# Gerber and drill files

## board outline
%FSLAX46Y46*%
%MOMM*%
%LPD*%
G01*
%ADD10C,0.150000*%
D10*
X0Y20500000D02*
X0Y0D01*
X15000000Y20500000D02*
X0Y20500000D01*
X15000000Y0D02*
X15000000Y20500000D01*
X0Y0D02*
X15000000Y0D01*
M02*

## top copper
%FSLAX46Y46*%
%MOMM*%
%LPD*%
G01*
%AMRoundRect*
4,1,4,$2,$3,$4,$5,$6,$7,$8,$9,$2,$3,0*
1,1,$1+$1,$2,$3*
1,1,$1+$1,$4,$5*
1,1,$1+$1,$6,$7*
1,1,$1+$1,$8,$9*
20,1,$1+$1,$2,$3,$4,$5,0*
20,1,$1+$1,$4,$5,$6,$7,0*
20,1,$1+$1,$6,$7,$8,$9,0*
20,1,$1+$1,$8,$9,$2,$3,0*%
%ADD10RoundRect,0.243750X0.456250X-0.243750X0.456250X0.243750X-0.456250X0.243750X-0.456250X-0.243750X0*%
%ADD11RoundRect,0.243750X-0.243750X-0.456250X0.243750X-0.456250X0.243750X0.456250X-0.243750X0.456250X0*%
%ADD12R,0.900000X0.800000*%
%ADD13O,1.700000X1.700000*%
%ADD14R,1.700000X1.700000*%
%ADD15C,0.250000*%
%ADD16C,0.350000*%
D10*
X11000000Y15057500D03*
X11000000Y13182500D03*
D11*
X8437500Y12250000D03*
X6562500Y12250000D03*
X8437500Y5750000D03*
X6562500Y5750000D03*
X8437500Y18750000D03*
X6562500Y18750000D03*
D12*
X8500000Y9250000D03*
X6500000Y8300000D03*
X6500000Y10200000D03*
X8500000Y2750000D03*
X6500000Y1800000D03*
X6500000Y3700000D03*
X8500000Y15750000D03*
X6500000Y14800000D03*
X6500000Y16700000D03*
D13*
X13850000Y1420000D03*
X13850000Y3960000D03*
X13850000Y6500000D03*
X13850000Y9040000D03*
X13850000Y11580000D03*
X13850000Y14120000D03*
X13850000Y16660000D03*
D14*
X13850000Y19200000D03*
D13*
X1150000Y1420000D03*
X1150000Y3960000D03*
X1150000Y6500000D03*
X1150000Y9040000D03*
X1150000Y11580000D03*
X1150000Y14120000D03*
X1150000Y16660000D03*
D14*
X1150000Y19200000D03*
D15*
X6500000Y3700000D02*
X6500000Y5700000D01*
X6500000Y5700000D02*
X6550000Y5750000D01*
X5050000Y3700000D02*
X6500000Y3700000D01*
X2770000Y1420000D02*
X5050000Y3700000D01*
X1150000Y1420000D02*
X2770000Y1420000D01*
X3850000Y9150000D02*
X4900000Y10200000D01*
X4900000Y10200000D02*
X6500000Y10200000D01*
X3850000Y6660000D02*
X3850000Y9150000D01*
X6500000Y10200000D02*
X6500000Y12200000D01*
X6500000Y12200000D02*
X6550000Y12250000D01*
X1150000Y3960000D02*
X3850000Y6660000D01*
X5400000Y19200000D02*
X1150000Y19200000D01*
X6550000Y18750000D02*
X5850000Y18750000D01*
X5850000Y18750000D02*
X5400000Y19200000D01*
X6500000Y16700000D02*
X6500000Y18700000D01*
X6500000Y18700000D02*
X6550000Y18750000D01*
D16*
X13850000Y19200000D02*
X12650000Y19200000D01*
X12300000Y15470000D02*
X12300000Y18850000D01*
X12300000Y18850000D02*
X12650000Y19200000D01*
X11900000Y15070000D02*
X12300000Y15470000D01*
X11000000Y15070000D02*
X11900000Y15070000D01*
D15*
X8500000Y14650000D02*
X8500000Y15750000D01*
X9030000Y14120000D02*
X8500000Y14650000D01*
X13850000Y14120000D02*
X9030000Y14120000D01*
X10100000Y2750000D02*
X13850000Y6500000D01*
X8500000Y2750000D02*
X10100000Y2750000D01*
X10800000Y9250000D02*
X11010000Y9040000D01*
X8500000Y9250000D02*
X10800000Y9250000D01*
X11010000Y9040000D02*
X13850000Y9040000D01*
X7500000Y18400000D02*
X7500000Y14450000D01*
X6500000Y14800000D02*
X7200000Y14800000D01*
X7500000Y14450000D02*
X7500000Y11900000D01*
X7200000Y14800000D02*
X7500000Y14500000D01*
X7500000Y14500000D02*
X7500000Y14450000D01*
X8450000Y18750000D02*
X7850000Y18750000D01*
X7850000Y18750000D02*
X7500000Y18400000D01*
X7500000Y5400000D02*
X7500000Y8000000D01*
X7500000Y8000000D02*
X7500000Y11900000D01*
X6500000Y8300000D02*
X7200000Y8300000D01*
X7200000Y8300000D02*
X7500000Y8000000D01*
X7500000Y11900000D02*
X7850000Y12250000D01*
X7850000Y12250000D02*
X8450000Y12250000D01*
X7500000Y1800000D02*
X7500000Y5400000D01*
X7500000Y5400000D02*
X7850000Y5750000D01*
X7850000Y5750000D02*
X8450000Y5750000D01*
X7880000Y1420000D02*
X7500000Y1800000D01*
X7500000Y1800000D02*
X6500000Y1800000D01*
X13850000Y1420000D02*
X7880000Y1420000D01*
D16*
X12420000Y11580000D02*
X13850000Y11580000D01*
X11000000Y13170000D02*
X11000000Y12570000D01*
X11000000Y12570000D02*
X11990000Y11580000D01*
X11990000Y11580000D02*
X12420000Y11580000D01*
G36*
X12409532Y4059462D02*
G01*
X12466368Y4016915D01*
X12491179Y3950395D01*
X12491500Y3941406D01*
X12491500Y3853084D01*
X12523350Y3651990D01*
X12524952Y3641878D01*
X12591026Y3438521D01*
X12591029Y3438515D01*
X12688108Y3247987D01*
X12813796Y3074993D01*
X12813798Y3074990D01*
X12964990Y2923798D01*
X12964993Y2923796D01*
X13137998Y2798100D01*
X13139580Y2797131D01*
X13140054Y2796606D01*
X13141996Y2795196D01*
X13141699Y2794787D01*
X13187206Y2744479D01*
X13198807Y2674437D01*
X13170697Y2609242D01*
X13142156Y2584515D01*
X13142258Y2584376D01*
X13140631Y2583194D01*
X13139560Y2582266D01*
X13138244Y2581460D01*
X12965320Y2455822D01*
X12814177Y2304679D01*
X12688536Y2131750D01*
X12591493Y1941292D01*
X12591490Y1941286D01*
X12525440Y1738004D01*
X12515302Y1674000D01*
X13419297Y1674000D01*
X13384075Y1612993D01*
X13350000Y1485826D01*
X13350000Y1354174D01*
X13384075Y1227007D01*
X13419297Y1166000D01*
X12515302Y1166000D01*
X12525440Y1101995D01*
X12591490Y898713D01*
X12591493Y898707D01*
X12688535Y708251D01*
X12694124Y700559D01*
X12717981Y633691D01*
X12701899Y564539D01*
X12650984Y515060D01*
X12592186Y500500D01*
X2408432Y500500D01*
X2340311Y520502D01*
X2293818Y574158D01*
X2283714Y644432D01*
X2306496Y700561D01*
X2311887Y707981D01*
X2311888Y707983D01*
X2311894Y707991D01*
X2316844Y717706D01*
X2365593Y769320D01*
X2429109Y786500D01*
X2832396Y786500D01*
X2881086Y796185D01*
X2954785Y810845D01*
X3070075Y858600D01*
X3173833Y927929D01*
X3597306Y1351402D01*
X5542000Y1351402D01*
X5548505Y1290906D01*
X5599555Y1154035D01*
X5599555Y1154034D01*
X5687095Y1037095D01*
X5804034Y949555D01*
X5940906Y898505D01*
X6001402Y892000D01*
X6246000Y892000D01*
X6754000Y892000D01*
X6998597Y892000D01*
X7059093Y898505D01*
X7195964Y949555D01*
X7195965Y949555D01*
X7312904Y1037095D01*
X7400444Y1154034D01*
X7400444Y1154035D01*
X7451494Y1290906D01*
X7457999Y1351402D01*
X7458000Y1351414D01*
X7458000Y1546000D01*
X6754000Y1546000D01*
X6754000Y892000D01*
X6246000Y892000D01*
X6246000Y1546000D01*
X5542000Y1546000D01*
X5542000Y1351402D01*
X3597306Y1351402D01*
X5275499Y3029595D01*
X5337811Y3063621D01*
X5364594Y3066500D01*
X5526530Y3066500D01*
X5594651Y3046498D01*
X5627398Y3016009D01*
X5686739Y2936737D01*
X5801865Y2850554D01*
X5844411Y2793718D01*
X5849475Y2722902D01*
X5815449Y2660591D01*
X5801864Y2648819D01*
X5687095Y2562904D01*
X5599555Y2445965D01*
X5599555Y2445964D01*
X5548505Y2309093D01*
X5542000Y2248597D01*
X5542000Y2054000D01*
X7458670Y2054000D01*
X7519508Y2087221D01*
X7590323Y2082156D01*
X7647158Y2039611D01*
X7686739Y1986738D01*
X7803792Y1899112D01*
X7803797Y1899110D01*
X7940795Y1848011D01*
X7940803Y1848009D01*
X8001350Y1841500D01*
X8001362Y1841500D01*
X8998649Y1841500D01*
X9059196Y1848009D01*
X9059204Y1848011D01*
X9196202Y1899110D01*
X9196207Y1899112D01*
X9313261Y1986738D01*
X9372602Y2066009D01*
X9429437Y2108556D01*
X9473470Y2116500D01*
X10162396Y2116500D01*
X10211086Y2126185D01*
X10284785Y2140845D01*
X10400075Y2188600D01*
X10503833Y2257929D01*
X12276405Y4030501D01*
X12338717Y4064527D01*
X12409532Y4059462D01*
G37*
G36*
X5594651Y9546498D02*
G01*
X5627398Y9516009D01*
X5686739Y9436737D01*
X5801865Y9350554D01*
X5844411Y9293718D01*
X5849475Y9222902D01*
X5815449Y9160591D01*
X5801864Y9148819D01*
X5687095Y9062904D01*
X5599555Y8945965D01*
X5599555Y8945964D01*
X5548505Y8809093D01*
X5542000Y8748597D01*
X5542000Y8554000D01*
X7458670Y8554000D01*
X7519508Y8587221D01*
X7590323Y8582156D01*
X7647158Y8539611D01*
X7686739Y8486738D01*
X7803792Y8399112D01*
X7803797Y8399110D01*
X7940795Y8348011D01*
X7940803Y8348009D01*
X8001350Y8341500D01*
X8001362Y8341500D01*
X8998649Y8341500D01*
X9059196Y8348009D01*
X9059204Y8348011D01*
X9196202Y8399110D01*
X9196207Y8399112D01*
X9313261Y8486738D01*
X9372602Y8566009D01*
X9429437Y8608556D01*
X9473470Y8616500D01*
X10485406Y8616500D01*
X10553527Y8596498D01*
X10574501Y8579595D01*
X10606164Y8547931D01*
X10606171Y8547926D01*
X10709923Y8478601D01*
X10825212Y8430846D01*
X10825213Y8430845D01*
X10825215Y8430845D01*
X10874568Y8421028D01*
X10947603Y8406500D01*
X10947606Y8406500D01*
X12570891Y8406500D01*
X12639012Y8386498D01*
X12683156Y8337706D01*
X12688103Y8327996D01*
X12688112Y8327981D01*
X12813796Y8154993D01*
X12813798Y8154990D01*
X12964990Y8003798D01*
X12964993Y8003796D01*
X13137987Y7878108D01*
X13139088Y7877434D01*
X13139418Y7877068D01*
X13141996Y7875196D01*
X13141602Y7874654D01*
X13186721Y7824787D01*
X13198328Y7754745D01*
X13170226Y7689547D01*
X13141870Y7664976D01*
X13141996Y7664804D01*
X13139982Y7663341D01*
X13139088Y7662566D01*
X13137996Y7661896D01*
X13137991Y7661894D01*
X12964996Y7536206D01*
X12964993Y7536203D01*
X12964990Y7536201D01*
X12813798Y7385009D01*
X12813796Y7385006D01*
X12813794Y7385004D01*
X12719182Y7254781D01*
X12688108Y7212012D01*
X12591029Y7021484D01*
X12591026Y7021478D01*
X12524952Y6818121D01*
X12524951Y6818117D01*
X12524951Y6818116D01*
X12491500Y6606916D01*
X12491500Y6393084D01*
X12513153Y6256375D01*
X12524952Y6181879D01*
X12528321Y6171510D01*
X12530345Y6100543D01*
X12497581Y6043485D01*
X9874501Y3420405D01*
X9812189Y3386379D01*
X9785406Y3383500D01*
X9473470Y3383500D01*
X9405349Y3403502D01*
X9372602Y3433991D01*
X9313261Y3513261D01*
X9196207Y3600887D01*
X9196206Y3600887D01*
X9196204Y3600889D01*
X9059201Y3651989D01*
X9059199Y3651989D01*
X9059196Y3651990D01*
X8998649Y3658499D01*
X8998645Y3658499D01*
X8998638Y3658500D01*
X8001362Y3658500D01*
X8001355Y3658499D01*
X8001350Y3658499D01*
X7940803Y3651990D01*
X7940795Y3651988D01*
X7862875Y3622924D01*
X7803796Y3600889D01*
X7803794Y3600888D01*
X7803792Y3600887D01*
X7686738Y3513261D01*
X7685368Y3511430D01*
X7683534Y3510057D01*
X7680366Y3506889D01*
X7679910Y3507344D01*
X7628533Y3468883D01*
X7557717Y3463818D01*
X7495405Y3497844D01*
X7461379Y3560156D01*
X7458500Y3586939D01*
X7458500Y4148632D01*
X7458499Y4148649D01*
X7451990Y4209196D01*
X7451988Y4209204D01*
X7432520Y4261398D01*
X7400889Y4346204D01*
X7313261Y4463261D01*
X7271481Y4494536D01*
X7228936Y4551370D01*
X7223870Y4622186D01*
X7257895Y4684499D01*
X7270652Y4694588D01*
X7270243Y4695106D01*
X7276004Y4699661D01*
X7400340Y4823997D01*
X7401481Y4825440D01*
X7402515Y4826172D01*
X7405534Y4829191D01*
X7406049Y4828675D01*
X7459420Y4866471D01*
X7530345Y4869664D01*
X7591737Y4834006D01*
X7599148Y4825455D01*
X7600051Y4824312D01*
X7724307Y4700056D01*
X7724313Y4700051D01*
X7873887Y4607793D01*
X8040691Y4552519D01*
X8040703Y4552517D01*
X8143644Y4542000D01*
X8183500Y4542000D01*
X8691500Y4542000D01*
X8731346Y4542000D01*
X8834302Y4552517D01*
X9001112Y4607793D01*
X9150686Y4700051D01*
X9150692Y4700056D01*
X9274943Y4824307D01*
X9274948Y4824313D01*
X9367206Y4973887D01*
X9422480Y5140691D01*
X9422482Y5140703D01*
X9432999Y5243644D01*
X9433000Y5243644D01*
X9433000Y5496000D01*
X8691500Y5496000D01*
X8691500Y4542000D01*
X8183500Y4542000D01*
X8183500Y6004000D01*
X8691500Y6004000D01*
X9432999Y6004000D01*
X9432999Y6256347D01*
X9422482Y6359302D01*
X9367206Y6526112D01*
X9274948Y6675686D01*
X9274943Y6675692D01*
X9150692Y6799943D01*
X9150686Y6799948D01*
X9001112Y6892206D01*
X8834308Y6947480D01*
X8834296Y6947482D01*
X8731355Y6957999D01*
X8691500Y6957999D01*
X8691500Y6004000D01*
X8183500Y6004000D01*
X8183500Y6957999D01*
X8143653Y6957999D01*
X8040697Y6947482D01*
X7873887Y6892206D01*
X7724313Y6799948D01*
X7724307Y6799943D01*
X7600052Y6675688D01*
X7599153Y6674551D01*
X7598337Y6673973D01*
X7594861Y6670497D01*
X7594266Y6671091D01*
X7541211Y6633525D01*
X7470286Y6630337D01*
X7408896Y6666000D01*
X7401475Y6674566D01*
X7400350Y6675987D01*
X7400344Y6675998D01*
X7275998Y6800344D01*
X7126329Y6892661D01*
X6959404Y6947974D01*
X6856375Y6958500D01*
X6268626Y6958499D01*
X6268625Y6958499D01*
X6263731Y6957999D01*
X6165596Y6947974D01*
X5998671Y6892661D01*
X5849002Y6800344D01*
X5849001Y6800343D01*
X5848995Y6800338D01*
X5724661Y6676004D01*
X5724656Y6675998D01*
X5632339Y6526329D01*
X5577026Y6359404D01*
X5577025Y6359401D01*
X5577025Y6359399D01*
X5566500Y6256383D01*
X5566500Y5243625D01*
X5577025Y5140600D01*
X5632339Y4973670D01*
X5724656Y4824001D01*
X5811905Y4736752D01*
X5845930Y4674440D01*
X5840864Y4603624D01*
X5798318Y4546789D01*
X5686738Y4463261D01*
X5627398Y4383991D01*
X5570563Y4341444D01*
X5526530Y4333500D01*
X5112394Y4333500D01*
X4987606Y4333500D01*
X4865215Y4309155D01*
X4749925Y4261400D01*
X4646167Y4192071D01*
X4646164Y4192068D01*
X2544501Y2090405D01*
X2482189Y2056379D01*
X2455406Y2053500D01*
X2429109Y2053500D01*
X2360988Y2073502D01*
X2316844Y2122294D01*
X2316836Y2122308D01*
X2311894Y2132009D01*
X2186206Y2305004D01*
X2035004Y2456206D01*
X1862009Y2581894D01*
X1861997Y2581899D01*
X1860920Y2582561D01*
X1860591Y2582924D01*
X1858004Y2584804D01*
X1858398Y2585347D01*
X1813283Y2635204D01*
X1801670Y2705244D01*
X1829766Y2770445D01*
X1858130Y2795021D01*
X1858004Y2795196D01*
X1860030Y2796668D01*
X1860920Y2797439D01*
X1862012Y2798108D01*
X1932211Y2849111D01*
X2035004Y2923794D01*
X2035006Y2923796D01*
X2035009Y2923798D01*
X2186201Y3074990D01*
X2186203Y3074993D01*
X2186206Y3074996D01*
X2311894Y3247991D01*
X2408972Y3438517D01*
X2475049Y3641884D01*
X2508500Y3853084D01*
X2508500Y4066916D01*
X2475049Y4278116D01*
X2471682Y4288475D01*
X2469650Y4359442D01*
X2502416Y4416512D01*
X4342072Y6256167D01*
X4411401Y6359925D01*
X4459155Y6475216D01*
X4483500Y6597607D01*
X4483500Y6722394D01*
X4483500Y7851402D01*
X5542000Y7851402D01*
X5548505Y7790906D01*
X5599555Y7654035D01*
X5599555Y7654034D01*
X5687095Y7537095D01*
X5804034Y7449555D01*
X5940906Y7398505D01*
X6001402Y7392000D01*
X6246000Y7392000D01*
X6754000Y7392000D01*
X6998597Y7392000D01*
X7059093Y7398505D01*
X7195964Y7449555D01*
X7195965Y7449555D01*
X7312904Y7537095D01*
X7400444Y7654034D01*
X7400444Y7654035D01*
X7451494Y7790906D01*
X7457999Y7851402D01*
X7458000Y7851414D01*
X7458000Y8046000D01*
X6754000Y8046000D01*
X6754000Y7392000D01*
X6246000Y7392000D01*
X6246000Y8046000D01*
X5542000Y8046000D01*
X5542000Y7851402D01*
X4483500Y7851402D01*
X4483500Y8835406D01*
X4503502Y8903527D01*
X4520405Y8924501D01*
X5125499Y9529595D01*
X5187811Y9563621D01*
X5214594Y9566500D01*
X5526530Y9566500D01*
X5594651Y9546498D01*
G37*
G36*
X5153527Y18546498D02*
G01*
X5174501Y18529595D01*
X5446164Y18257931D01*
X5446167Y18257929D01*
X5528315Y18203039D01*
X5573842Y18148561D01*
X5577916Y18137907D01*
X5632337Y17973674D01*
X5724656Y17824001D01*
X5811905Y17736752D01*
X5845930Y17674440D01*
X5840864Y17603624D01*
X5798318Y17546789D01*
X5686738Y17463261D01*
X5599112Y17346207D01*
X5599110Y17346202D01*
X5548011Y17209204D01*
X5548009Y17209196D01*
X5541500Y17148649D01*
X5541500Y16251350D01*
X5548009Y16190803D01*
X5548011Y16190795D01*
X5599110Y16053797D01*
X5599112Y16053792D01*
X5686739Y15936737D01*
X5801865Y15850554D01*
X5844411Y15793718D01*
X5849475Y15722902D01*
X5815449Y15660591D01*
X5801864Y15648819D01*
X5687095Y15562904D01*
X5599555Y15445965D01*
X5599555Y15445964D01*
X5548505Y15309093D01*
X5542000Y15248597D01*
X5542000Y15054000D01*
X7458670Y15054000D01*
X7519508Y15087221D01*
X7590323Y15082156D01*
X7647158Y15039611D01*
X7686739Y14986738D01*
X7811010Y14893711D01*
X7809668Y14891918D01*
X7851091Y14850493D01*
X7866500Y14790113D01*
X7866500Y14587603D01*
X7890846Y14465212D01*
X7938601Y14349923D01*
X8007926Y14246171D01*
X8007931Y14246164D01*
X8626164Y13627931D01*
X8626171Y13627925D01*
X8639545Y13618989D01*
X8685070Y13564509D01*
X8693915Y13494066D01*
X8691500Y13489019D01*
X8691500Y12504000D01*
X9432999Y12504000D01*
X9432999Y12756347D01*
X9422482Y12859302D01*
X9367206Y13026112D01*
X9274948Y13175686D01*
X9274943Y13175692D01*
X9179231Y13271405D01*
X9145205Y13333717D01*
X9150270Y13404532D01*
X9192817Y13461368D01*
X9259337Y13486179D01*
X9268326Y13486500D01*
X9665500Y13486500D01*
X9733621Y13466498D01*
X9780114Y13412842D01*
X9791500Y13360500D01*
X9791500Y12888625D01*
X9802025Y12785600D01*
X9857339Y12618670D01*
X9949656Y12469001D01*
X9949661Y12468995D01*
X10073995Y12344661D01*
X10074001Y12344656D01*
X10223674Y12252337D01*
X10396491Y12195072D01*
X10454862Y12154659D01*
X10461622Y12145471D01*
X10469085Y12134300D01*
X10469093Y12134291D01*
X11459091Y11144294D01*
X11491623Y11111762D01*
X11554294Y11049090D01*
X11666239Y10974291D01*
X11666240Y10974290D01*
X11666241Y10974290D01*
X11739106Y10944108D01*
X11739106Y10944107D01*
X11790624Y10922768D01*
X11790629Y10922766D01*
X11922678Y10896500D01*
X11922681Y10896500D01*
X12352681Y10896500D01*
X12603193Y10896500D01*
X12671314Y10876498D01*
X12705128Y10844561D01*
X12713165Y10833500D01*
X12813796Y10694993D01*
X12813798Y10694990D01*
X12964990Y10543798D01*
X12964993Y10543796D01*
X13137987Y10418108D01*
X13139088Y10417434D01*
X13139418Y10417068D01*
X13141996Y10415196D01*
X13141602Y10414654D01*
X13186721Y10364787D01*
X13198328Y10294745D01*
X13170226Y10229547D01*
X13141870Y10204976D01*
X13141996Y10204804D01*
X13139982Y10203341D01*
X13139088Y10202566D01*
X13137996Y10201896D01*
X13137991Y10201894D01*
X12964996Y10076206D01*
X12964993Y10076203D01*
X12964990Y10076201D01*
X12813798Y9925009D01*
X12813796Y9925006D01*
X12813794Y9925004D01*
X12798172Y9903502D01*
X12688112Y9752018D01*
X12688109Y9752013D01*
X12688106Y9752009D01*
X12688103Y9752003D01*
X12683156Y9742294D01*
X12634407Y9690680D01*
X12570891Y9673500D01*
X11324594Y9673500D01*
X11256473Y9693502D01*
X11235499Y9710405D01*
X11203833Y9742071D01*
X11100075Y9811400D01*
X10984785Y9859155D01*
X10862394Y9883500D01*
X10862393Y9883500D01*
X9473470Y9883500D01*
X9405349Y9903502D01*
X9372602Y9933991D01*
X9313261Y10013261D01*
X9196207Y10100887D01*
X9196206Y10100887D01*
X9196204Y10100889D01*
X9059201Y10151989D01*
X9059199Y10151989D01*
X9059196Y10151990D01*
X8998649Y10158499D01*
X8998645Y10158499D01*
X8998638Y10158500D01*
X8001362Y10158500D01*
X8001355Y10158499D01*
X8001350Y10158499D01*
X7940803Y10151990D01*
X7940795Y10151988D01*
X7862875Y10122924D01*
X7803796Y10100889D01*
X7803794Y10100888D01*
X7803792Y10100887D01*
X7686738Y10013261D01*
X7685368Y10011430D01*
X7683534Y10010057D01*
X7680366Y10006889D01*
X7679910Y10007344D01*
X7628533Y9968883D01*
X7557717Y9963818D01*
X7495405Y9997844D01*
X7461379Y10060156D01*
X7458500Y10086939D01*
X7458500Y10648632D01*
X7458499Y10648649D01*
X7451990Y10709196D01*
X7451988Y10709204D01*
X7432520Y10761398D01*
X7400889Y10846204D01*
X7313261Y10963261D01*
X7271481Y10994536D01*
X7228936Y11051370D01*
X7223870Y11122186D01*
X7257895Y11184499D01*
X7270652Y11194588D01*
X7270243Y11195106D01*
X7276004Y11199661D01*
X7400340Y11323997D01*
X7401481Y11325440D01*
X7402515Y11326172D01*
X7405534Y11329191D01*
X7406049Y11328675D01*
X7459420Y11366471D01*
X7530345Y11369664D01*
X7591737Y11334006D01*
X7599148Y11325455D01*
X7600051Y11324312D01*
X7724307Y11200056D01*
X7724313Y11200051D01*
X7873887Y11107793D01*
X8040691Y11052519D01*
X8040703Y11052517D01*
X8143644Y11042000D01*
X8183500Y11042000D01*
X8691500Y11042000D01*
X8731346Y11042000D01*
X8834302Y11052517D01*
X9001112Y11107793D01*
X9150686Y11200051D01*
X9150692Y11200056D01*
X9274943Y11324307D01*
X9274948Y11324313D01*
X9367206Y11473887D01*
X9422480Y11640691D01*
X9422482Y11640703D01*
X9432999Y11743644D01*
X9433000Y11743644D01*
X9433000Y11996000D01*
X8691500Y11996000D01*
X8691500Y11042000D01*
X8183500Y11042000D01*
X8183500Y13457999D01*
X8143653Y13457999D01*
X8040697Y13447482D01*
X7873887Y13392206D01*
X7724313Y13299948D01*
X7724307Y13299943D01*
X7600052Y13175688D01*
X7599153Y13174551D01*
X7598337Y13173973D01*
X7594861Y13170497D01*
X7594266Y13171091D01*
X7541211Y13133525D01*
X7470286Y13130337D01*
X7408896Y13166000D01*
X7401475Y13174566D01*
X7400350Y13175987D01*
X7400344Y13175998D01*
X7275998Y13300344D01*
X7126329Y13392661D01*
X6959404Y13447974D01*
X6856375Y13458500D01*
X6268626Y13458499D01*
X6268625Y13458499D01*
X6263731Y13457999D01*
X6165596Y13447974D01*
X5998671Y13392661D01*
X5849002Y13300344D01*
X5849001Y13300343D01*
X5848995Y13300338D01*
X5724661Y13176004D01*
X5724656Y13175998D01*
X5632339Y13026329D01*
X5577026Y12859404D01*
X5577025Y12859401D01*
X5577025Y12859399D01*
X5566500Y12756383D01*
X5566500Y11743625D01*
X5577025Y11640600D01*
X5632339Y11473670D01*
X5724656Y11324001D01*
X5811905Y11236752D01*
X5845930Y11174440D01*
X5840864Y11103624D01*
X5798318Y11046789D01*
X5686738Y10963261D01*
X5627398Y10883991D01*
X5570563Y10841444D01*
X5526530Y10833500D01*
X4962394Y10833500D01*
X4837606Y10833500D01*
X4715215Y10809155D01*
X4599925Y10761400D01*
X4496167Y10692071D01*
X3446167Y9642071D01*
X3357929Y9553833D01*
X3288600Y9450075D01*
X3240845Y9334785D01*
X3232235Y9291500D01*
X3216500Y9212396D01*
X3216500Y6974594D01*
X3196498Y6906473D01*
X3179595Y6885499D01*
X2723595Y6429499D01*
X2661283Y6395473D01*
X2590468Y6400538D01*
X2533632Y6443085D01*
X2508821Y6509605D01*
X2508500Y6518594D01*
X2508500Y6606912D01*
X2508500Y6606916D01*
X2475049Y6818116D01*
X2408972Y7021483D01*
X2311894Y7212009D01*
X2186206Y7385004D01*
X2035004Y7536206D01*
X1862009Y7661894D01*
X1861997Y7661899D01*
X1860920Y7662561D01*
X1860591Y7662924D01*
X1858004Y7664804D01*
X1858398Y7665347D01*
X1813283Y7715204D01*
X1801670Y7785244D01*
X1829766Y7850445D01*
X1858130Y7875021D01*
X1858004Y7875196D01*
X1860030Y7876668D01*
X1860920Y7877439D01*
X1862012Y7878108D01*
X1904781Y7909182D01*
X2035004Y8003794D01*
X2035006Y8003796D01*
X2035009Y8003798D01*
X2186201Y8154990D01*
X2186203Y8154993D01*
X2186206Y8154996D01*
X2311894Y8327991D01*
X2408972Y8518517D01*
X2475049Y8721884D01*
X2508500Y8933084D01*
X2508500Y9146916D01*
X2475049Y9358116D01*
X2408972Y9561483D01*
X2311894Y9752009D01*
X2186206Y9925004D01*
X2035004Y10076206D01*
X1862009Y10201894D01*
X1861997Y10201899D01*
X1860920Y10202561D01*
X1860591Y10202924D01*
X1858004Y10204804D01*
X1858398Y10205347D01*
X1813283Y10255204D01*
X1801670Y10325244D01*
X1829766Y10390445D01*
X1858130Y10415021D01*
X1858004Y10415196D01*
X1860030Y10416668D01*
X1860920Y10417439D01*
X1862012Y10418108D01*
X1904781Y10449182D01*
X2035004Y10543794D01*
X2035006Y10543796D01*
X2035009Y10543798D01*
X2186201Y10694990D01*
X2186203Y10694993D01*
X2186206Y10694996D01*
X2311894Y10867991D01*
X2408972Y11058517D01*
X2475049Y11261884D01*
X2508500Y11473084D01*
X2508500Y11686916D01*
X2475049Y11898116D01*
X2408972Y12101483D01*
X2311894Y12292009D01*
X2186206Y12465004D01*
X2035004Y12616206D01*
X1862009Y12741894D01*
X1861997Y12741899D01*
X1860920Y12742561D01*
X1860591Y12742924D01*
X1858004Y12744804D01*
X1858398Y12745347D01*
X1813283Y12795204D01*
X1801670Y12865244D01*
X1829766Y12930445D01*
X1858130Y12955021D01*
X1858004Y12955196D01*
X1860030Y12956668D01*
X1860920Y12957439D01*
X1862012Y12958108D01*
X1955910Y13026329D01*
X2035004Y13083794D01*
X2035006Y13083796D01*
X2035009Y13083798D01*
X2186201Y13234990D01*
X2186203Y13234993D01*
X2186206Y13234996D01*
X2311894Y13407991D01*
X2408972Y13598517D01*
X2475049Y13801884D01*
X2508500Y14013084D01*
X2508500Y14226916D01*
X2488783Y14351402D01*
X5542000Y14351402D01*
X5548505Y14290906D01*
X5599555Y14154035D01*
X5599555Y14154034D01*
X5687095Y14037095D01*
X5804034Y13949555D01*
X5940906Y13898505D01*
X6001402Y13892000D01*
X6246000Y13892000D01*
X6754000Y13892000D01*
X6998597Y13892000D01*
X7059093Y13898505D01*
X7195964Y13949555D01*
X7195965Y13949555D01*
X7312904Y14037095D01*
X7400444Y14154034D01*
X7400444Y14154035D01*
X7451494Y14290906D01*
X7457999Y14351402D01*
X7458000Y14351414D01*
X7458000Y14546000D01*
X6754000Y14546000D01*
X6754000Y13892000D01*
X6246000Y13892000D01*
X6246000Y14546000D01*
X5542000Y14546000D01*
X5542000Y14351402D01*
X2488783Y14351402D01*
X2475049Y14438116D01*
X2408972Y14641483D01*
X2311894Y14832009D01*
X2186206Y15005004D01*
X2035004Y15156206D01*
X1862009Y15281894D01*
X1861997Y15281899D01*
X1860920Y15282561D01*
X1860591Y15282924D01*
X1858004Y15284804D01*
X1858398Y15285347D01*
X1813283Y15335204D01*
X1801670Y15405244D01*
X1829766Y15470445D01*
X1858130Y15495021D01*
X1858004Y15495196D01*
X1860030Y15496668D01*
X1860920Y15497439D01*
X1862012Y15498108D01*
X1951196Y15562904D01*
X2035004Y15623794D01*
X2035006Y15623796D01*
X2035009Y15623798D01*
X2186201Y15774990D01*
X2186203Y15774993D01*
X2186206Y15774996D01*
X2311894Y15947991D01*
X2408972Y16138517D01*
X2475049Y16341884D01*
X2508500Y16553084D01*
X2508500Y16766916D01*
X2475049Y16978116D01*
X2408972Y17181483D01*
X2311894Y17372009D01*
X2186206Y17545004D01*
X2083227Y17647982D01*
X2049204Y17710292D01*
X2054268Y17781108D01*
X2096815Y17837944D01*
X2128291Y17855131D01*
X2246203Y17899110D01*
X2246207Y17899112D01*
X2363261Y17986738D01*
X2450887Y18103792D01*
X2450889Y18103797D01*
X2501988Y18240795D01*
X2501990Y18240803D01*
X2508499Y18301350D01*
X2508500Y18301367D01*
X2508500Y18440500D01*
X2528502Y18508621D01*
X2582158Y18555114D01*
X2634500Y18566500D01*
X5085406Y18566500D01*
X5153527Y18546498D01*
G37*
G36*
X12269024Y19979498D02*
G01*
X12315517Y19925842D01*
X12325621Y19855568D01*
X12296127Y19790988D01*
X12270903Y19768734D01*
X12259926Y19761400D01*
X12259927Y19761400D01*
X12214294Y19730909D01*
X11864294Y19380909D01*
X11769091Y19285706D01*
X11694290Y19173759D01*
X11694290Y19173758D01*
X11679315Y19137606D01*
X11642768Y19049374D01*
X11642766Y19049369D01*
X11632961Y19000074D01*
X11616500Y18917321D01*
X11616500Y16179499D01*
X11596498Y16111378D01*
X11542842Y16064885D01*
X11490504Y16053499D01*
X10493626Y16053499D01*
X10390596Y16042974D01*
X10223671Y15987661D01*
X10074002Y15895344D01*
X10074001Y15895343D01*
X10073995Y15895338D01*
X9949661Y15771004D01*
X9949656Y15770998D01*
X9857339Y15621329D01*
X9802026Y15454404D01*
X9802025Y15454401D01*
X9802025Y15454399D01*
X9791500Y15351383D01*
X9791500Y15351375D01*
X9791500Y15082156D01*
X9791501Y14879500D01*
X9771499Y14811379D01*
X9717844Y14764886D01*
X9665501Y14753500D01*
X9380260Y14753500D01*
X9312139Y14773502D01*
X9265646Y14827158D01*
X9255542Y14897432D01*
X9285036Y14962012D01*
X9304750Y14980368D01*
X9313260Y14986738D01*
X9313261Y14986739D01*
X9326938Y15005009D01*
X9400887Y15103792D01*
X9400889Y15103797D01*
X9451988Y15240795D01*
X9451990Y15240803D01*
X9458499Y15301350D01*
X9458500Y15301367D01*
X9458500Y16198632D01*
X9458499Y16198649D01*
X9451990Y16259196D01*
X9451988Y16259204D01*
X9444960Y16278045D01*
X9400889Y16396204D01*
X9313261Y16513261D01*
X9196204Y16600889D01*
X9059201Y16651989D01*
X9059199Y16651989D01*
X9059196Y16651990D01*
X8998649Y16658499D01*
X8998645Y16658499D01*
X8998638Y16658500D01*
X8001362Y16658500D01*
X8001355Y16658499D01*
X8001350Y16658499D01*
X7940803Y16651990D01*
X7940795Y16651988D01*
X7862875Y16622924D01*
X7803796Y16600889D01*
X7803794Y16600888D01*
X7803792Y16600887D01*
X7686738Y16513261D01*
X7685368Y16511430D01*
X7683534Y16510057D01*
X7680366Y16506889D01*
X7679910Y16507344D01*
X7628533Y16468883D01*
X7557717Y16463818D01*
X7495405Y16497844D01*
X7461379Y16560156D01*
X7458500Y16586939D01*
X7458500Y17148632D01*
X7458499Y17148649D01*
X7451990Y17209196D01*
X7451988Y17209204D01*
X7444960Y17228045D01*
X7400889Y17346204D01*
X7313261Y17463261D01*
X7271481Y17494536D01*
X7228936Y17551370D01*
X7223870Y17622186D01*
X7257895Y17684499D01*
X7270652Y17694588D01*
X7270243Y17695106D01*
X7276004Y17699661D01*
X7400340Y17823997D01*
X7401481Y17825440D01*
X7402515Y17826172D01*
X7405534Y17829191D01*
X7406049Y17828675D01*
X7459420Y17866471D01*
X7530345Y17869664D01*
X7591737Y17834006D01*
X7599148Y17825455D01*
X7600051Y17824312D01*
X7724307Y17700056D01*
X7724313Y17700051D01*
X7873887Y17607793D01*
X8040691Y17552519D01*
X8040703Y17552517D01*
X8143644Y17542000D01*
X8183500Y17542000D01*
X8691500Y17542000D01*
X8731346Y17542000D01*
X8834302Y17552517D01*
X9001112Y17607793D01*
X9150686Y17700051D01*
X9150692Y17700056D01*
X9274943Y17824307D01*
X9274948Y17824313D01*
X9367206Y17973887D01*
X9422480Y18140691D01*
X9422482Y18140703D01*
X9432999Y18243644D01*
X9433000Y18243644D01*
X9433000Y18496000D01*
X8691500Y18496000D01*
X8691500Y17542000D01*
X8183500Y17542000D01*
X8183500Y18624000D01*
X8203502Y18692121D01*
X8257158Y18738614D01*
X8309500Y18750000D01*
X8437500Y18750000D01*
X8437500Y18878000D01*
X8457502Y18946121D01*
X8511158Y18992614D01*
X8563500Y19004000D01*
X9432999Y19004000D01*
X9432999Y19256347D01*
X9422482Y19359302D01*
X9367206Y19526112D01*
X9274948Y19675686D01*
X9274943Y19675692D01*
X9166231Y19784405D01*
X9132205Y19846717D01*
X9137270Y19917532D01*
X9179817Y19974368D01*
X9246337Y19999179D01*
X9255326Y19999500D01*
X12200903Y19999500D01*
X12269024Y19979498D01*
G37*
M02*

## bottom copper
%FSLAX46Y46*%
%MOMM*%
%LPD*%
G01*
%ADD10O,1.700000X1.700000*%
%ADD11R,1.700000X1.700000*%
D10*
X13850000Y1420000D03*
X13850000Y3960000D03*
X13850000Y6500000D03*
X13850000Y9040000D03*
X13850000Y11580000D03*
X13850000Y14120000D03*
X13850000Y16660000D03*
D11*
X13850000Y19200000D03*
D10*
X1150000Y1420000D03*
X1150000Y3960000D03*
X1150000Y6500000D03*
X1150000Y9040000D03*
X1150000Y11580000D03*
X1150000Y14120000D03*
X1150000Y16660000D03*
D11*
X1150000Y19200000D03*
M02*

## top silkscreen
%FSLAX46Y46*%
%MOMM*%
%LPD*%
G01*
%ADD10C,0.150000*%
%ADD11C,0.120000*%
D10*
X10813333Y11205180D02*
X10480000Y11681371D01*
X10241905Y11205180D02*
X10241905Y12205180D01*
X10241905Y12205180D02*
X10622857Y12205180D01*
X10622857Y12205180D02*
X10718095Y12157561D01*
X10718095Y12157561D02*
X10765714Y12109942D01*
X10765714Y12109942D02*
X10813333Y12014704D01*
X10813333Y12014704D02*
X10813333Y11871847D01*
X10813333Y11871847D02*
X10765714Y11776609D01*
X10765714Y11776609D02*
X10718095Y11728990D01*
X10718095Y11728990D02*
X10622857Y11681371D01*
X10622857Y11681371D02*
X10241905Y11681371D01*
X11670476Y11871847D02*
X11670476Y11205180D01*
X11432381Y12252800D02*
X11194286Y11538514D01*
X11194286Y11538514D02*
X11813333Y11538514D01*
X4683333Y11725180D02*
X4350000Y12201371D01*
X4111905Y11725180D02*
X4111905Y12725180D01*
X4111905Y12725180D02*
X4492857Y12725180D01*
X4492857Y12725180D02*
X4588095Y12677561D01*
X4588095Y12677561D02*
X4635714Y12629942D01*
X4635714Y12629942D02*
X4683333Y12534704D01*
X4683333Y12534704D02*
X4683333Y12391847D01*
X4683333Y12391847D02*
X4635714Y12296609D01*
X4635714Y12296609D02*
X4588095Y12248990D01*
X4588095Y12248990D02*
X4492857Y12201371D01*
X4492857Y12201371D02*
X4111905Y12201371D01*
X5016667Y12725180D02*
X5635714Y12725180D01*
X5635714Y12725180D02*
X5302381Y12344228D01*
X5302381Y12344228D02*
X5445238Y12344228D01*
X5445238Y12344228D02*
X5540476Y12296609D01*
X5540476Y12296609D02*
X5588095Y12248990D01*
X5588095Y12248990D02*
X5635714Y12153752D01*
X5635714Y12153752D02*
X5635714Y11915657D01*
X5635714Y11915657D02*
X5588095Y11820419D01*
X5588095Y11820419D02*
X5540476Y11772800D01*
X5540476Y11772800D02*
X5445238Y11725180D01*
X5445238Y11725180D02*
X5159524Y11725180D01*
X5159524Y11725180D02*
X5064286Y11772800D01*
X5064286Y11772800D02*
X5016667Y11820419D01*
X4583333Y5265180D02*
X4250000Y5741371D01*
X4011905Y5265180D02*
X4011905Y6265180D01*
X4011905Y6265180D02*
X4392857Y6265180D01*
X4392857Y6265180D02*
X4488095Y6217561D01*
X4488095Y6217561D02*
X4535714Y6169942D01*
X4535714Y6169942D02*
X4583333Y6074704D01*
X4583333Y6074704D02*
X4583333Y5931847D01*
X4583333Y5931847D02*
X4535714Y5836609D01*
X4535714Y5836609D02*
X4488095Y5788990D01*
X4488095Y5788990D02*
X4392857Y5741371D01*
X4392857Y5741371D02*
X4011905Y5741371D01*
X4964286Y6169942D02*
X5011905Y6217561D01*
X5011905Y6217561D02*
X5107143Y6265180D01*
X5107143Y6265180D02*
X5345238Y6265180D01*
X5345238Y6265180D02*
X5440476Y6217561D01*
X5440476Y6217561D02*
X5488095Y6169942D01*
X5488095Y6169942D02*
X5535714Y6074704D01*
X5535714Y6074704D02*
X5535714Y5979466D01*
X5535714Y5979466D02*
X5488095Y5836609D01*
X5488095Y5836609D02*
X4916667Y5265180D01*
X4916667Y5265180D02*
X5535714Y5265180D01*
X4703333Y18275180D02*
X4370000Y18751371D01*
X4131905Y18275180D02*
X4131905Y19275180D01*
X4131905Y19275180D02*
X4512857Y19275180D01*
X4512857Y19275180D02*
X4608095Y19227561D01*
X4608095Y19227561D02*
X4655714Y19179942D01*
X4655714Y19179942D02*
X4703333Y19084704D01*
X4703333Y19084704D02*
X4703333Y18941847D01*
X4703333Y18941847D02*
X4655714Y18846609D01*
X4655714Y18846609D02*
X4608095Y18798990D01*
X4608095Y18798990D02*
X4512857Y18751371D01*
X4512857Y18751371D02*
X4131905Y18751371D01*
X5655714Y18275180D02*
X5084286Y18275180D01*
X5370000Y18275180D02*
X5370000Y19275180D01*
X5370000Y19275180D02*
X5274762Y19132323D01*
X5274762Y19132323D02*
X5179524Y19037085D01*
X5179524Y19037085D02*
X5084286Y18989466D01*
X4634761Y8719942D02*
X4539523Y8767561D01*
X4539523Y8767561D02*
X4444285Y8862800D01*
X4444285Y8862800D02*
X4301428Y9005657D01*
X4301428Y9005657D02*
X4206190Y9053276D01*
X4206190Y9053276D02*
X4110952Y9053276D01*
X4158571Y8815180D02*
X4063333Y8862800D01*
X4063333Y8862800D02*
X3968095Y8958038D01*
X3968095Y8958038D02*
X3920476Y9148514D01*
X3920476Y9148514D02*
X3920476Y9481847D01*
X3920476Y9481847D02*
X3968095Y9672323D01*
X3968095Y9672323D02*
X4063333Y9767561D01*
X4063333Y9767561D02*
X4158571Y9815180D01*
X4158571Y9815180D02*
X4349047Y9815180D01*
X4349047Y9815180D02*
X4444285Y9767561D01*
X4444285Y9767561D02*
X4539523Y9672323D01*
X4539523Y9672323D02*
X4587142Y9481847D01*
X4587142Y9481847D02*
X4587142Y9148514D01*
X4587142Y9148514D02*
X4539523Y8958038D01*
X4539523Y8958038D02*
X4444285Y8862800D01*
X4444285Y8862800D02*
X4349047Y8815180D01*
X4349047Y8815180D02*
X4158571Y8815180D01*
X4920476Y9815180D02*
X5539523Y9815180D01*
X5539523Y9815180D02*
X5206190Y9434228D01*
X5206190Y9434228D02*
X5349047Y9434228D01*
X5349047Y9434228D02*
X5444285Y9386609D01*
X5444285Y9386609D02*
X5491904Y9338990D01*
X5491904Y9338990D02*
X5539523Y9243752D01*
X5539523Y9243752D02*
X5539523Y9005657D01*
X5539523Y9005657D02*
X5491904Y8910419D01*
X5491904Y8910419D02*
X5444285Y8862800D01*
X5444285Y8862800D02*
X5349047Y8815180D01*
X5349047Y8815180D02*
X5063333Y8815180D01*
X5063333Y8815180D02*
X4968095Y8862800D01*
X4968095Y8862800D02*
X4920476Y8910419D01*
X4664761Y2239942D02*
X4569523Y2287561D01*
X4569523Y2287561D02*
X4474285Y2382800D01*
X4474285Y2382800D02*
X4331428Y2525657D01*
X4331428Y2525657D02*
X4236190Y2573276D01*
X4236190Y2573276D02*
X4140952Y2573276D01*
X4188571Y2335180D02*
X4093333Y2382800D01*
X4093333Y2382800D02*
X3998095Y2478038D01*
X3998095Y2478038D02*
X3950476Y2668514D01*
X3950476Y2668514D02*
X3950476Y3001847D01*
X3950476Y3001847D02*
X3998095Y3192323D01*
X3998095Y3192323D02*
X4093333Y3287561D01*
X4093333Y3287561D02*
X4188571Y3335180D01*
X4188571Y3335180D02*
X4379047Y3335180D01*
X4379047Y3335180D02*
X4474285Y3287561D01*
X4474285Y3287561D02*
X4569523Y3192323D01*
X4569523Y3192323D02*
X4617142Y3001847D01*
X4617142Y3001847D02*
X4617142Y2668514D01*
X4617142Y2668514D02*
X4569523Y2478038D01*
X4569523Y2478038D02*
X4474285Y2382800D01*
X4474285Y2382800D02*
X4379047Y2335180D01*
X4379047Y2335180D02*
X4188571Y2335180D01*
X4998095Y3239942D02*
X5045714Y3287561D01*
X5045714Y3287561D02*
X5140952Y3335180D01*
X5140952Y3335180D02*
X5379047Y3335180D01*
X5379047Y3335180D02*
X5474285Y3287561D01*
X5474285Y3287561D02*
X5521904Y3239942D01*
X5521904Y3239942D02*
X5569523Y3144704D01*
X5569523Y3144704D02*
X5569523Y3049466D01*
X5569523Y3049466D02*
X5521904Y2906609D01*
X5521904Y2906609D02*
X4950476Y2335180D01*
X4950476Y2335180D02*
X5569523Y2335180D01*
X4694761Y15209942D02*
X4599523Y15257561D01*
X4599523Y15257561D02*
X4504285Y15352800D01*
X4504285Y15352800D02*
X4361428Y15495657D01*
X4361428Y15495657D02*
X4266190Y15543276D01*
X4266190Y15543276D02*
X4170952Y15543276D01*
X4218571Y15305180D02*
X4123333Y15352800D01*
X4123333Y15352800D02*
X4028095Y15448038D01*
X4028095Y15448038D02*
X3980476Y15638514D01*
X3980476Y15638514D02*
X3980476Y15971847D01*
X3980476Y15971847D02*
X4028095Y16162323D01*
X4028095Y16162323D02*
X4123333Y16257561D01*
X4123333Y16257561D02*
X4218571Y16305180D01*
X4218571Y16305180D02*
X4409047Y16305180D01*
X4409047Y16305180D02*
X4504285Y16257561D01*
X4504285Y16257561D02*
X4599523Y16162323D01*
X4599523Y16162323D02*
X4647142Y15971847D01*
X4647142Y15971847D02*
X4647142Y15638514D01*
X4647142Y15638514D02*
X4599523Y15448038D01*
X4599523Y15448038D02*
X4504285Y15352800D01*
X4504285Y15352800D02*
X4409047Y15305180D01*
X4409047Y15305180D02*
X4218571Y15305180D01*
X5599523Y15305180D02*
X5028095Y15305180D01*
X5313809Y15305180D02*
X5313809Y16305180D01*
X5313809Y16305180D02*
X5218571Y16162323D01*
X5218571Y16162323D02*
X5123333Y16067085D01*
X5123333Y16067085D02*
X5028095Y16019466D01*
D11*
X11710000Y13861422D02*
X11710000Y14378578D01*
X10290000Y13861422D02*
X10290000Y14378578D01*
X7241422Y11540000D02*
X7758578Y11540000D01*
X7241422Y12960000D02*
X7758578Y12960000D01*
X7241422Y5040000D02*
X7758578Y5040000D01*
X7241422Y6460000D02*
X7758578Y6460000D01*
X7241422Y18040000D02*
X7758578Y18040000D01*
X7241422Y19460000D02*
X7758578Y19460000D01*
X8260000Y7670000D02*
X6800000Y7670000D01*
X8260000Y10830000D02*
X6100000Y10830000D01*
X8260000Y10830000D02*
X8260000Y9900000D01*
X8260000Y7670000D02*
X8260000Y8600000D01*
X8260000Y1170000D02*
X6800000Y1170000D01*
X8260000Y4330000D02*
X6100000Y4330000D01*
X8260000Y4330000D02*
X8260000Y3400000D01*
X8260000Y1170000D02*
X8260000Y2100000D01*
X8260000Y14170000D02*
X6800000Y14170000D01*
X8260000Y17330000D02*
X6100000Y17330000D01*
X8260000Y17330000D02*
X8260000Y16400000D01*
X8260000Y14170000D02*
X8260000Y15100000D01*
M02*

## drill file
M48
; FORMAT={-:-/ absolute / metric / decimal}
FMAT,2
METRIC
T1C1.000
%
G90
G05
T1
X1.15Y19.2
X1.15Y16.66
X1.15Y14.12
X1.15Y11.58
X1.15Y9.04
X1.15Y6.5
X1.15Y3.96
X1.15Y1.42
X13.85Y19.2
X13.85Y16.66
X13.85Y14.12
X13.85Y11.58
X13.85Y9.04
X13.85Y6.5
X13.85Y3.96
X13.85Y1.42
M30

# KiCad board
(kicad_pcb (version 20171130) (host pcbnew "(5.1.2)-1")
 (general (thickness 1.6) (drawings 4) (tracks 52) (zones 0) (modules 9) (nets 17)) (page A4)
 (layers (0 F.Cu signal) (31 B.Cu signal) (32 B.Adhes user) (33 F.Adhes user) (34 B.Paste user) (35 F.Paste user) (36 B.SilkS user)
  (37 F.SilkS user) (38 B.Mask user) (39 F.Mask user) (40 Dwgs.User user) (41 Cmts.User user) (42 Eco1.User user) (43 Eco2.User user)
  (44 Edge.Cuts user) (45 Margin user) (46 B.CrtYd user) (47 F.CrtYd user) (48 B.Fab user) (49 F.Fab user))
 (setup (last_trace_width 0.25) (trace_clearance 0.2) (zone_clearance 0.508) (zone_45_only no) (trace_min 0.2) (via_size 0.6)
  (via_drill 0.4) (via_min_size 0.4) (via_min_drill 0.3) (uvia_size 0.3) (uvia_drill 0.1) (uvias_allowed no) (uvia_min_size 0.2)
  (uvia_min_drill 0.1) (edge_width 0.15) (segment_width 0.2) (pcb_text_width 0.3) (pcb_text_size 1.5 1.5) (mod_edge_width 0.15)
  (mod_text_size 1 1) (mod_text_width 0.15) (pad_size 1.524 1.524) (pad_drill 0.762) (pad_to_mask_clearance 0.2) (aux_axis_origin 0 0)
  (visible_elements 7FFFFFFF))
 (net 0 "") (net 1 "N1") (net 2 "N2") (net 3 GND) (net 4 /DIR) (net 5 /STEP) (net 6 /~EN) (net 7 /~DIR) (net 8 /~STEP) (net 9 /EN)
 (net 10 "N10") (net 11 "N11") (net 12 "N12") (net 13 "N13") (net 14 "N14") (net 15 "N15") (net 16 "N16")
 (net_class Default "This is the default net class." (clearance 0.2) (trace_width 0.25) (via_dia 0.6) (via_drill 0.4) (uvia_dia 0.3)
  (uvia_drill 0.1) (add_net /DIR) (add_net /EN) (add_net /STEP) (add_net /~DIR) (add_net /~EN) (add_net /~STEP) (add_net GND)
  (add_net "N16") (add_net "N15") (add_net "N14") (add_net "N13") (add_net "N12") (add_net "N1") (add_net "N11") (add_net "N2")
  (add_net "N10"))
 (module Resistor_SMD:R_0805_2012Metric (layer F.Cu) (at 11 -14.12 90)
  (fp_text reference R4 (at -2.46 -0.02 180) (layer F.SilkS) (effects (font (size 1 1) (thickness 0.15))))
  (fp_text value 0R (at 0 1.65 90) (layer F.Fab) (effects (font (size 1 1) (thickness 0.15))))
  (fp_line (start -0.258578 0.71) (end 0.258578 0.71) (layer F.SilkS) (width 0.12))
  (fp_line (start -0.258578 -0.71) (end 0.258578 -0.71) (layer F.SilkS) (width 0.12))
  (pad 2 smd roundrect (at 0.9375 0 90) (size 0.975 1.4) (layers F.Cu F.Paste F.Mask) (roundrect_rratio 0.25) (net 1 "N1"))
  (pad 1 smd roundrect (at -0.9375 0 90) (size 0.975 1.4) (layers F.Cu F.Paste F.Mask) (roundrect_rratio 0.25) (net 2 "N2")))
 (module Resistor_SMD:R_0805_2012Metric (layer F.Cu) (at 7.5 -12.25)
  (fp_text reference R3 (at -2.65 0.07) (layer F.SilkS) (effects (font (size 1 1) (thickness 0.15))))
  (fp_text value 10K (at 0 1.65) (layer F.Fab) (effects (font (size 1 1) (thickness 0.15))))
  (fp_line (start -0.258578 0.71) (end 0.258578 0.71) (layer F.SilkS) (width 0.12))
  (fp_line (start -0.258578 -0.71) (end 0.258578 -0.71) (layer F.SilkS) (width 0.12))
  (pad 2 smd roundrect (at 0.9375 0) (size 0.975 1.4) (layers F.Cu F.Paste F.Mask) (roundrect_rratio 0.25) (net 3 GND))
  (pad 1 smd roundrect (at -0.9375 0) (size 0.975 1.4) (layers F.Cu F.Paste F.Mask) (roundrect_rratio 0.25) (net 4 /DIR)))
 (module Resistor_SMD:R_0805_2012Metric (layer F.Cu) (at 7.5 -5.75)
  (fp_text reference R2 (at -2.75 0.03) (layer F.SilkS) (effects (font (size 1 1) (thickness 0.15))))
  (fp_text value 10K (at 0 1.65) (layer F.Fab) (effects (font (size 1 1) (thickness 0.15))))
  (fp_line (start -0.258578 0.71) (end 0.258578 0.71) (layer F.SilkS) (width 0.12))
  (fp_line (start -0.258578 -0.71) (end 0.258578 -0.71) (layer F.SilkS) (width 0.12))
  (pad 2 smd roundrect (at 0.9375 0) (size 0.975 1.4) (layers F.Cu F.Paste F.Mask) (roundrect_rratio 0.25) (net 3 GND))
  (pad 1 smd roundrect (at -0.9375 0) (size 0.975 1.4) (layers F.Cu F.Paste F.Mask) (roundrect_rratio 0.25) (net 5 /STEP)))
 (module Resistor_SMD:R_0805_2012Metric (layer F.Cu) (at 7.5 -18.75)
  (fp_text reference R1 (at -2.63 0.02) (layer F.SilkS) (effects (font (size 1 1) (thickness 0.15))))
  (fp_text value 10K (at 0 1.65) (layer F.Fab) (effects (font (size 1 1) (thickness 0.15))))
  (fp_line (start -0.258578 0.71) (end 0.258578 0.71) (layer F.SilkS) (width 0.12))
  (fp_line (start -0.258578 -0.71) (end 0.258578 -0.71) (layer F.SilkS) (width 0.12))
  (pad 2 smd roundrect (at 0.9375 0) (size 0.975 1.4) (layers F.Cu F.Paste F.Mask) (roundrect_rratio 0.25) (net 3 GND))
  (pad 1 smd roundrect (at -0.9375 0) (size 0.975 1.4) (layers F.Cu F.Paste F.Mask) (roundrect_rratio 0.25) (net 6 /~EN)))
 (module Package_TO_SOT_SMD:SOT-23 (layer F.Cu) (at 7.5 -9.25)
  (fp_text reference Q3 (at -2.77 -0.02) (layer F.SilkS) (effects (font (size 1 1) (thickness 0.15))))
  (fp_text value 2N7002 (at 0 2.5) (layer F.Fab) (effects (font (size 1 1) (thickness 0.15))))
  (fp_line (start 0.76 1.58) (end -0.7 1.58) (layer F.SilkS) (width 0.12))
  (fp_line (start 0.76 -1.58) (end -1.4 -1.58) (layer F.SilkS) (width 0.12))
  (fp_line (start 0.76 -1.58) (end 0.76 -0.65) (layer F.SilkS) (width 0.12))
  (fp_line (start 0.76 1.58) (end 0.76 0.65) (layer F.SilkS) (width 0.12))
  (pad 3 smd rect (at 1 0) (size 0.9 0.8) (layers F.Cu F.Paste F.Mask) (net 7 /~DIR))
  (pad 2 smd rect (at -1 0.95) (size 0.9 0.8) (layers F.Cu F.Paste F.Mask) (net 3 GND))
  (pad 1 smd rect (at -1 -0.95) (size 0.9 0.8) (layers F.Cu F.Paste F.Mask) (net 4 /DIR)))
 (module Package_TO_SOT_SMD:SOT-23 (layer F.Cu) (at 7.5 -2.75)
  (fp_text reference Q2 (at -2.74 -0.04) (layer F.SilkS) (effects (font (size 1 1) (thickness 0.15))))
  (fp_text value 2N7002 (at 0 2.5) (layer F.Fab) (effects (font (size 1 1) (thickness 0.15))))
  (fp_line (start 0.76 1.58) (end -0.7 1.58) (layer F.SilkS) (width 0.12))
  (fp_line (start 0.76 -1.58) (end -1.4 -1.58) (layer F.SilkS) (width 0.12))
  (fp_line (start 0.76 -1.58) (end 0.76 -0.65) (layer F.SilkS) (width 0.12))
  (fp_line (start 0.76 1.58) (end 0.76 0.65) (layer F.SilkS) (width 0.12))
  (pad 3 smd rect (at 1 0) (size 0.9 0.8) (layers F.Cu F.Paste F.Mask) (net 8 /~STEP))
  (pad 2 smd rect (at -1 0.95) (size 0.9 0.8) (layers F.Cu F.Paste F.Mask) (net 3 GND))
  (pad 1 smd rect (at -1 -0.95) (size 0.9 0.8) (layers F.Cu F.Paste F.Mask) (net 5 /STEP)))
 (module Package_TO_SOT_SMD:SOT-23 (layer F.Cu) (at 7.5 -15.75)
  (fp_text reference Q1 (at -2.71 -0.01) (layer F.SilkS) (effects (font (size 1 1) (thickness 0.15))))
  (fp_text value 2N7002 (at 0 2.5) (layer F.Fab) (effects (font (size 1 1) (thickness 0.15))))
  (fp_line (start 0.76 1.58) (end -0.7 1.58) (layer F.SilkS) (width 0.12))
  (fp_line (start 0.76 -1.58) (end -1.4 -1.58) (layer F.SilkS) (width 0.12))
  (fp_line (start 0.76 -1.58) (end 0.76 -0.65) (layer F.SilkS) (width 0.12))
  (fp_line (start 0.76 1.58) (end 0.76 0.65) (layer F.SilkS) (width 0.12))
  (pad 3 smd rect (at 1 0) (size 0.9 0.8) (layers F.Cu F.Paste F.Mask) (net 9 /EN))
  (pad 2 smd rect (at -1 0.95) (size 0.9 0.8) (layers F.Cu F.Paste F.Mask) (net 3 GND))
  (pad 1 smd rect (at -1 -0.95) (size 0.9 0.8) (layers F.Cu F.Paste F.Mask) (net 6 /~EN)))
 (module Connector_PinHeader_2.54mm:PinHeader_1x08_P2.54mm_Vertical (layer B.Cu) (at 13.85 -19.2 180)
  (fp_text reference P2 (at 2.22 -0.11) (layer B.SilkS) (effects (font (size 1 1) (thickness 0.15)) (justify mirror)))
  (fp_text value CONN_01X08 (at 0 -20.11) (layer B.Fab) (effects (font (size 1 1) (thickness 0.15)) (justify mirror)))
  (pad 8 thru_hole oval (at 0 -17.78 180) (size 1.7 1.7) (drill 1) (layers *.Cu *.Mask) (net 3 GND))
  (pad 7 thru_hole oval (at 0 -15.24 180) (size 1.7 1.7) (drill 1) (layers *.Cu *.Mask) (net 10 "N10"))
  (pad 6 thru_hole oval (at 0 -12.7 180) (size 1.7 1.7) (drill 1) (layers *.Cu *.Mask) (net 8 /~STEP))
  (pad 5 thru_hole oval (at 0 -10.16 180) (size 1.7 1.7) (drill 1) (layers *.Cu *.Mask) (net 7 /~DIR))
  (pad 4 thru_hole oval (at 0 -7.62 180) (size 1.7 1.7) (drill 1) (layers *.Cu *.Mask) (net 2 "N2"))
  (pad 3 thru_hole oval (at 0 -5.08 180) (size 1.7 1.7) (drill 1) (layers *.Cu *.Mask) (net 9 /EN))
  (pad 2 thru_hole oval (at 0 -2.54 180) (size 1.7 1.7) (drill 1) (layers *.Cu *.Mask) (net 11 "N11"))
  (pad 1 thru_hole rect (at 0 0 180) (size 1.7 1.7) (drill 1) (layers *.Cu *.Mask) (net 1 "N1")))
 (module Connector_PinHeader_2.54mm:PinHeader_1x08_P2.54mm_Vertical (layer B.Cu) (at 1.15 -19.2 180)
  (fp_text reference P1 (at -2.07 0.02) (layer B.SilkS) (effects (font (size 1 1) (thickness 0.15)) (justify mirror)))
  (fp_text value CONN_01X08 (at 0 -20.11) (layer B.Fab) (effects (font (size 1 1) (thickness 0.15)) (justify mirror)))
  (pad 8 thru_hole oval (at 0 -17.78 180) (size 1.7 1.7) (drill 1) (layers *.Cu *.Mask) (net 5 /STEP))
  (pad 7 thru_hole oval (at 0 -15.24 180) (size 1.7 1.7) (drill 1) (layers *.Cu *.Mask) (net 4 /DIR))
  (pad 6 thru_hole oval (at 0 -12.7 180) (size 1.7 1.7) (drill 1) (layers *.Cu *.Mask) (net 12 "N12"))
  (pad 5 thru_hole oval (at 0 -10.16 180) (size 1.7 1.7) (drill 1) (layers *.Cu *.Mask) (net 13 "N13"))
  (pad 4 thru_hole oval (at 0 -7.62 180) (size 1.7 1.7) (drill 1) (layers *.Cu *.Mask) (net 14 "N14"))
  (pad 3 thru_hole oval (at 0 -5.08 180) (size 1.7 1.7) (drill 1) (layers *.Cu *.Mask) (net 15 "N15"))
  (pad 2 thru_hole oval (at 0 -2.54 180) (size 1.7 1.7) (drill 1) (layers *.Cu *.Mask) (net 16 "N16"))
  (pad 1 thru_hole rect (at 0 0 180) (size 1.7 1.7) (drill 1) (layers *.Cu *.Mask) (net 6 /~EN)))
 (gr_line (start 0 -20.5) (end 0 0) (layer Edge.Cuts) (width 0.15))
 (gr_line (start 15 -20.5) (end 0 -20.5) (layer Edge.Cuts) (width 0.15))
 (gr_line (start 15 0) (end 15 -20.5) (layer Edge.Cuts) (width 0.15))
 (gr_line (start 0 0) (end 15 0) (layer Edge.Cuts) (width 0.15))
 (segment (start 6.5 -3.7) (end 6.5 -5.7) (width 0.25) (layer F.Cu) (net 5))
 (segment (start 6.5 -5.7) (end 6.55 -5.75) (width 0.25) (layer F.Cu) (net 5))
 (segment (start 5.05 -3.7) (end 6.5 -3.7) (width 0.25) (layer F.Cu) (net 5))
 (segment (start 2.77 -1.42) (end 5.05 -3.7) (width 0.25) (layer F.Cu) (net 5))
 (segment (start 1.15 -1.42) (end 2.77 -1.42) (width 0.25) (layer F.Cu) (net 5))
 (segment (start 3.85 -9.15) (end 4.9 -10.2) (width 0.25) (layer F.Cu) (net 4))
 (segment (start 4.9 -10.2) (end 6.5 -10.2) (width 0.25) (layer F.Cu) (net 4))
 (segment (start 3.85 -6.66) (end 3.85 -9.15) (width 0.25) (layer F.Cu) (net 4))
 (segment (start 6.5 -10.2) (end 6.5 -12.2) (width 0.25) (layer F.Cu) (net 4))
 (segment (start 6.5 -12.2) (end 6.55 -12.25) (width 0.25) (layer F.Cu) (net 4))
 (segment (start 1.15 -3.96) (end 3.85 -6.66) (width 0.25) (layer F.Cu) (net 4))
 (segment (start 5.4 -19.2) (end 1.15 -19.2) (width 0.25) (layer F.Cu) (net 6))
 (segment (start 6.55 -18.75) (end 5.85 -18.75) (width 0.25) (layer F.Cu) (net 6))
 (segment (start 5.85 -18.75) (end 5.4 -19.2) (width 0.25) (layer F.Cu) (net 6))
 (segment (start 6.5 -16.7) (end 6.5 -18.7) (width 0.25) (layer F.Cu) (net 6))
 (segment (start 6.5 -18.7) (end 6.55 -18.75) (width 0.25) (layer F.Cu) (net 6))
 (segment (start 13.85 -19.2) (end 12.65 -19.2) (width 0.35) (layer F.Cu) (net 1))
 (segment (start 12.3 -15.47) (end 12.3 -18.85) (width 0.35) (layer F.Cu) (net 1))
 (segment (start 12.3 -18.85) (end 12.65 -19.2) (width 0.35) (layer F.Cu) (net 1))
 (segment (start 11.9 -15.07) (end 12.3 -15.47) (width 0.35) (layer F.Cu) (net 1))
 (segment (start 11 -15.07) (end 11.9 -15.07) (width 0.35) (layer F.Cu) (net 1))
 (segment (start 8.5 -14.65) (end 8.5 -15.75) (width 0.25) (layer F.Cu) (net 9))
 (segment (start 9.03 -14.12) (end 8.5 -14.65) (width 0.25) (layer F.Cu) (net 9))
 (segment (start 13.85 -14.12) (end 9.03 -14.12) (width 0.25) (layer F.Cu) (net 9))
 (segment (start 10.1 -2.75) (end 13.85 -6.5) (width 0.25) (layer F.Cu) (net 8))
 (segment (start 8.5 -2.75) (end 10.1 -2.75) (width 0.25) (layer F.Cu) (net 8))
 (segment (start 10.8 -9.25) (end 11.01 -9.04) (width 0.25) (layer F.Cu) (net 7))
 (segment (start 8.5 -9.25) (end 10.8 -9.25) (width 0.25) (layer F.Cu) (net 7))
 (segment (start 11.01 -9.04) (end 13.85 -9.04) (width 0.25) (layer F.Cu) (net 7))
 (segment (start 7.5 -18.4) (end 7.5 -14.45) (width 0.25) (layer F.Cu) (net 3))
 (segment (start 6.5 -14.8) (end 7.2 -14.8) (width 0.25) (layer F.Cu) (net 3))
 (segment (start 7.5 -14.45) (end 7.5 -11.9) (width 0.25) (layer F.Cu) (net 3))
 (segment (start 7.2 -14.8) (end 7.5 -14.5) (width 0.25) (layer F.Cu) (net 3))
 (segment (start 7.5 -14.5) (end 7.5 -14.45) (width 0.25) (layer F.Cu) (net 3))
 (segment (start 8.45 -18.75) (end 7.85 -18.75) (width 0.25) (layer F.Cu) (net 3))
 (segment (start 7.85 -18.75) (end 7.5 -18.4) (width 0.25) (layer F.Cu) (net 3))
 (segment (start 7.5 -5.4) (end 7.5 -8) (width 0.25) (layer F.Cu) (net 3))
 (segment (start 7.5 -8) (end 7.5 -11.9) (width 0.25) (layer F.Cu) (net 3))
 (segment (start 6.5 -8.3) (end 7.2 -8.3) (width 0.25) (layer F.Cu) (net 3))
 (segment (start 7.2 -8.3) (end 7.5 -8) (width 0.25) (layer F.Cu) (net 3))
 (segment (start 7.5 -11.9) (end 7.85 -12.25) (width 0.25) (layer F.Cu) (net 3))
 (segment (start 7.85 -12.25) (end 8.45 -12.25) (width 0.25) (layer F.Cu) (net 3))
 (segment (start 7.5 -1.8) (end 7.5 -5.4) (width 0.25) (layer F.Cu) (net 3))
 (segment (start 7.5 -5.4) (end 7.85 -5.75) (width 0.25) (layer F.Cu) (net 3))
 (segment (start 7.85 -5.75) (end 8.45 -5.75) (width 0.25) (layer F.Cu) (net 3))
 (segment (start 7.88 -1.42) (end 7.5 -1.8) (width 0.25) (layer F.Cu) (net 3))
 (segment (start 7.5 -1.8) (end 6.5 -1.8) (width 0.25) (layer F.Cu) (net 3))
 (segment (start 13.85 -1.42) (end 7.88 -1.42) (width 0.25) (layer F.Cu) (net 3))
 (segment (start 12.42 -11.58) (end 13.85 -11.58) (width 0.35) (layer F.Cu) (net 2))
 (segment (start 11 -13.17) (end 11 -12.57) (width 0.35) (layer F.Cu) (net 2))
 (segment (start 11 -12.57) (end 11.99 -11.58) (width 0.35) (layer F.Cu) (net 2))
 (segment (start 11.99 -11.58) (end 12.42 -11.58) (width 0.35) (layer F.Cu) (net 2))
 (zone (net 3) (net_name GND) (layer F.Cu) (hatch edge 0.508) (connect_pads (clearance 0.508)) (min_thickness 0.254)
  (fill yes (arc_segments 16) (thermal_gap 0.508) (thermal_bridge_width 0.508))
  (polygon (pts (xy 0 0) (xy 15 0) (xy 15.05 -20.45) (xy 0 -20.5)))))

